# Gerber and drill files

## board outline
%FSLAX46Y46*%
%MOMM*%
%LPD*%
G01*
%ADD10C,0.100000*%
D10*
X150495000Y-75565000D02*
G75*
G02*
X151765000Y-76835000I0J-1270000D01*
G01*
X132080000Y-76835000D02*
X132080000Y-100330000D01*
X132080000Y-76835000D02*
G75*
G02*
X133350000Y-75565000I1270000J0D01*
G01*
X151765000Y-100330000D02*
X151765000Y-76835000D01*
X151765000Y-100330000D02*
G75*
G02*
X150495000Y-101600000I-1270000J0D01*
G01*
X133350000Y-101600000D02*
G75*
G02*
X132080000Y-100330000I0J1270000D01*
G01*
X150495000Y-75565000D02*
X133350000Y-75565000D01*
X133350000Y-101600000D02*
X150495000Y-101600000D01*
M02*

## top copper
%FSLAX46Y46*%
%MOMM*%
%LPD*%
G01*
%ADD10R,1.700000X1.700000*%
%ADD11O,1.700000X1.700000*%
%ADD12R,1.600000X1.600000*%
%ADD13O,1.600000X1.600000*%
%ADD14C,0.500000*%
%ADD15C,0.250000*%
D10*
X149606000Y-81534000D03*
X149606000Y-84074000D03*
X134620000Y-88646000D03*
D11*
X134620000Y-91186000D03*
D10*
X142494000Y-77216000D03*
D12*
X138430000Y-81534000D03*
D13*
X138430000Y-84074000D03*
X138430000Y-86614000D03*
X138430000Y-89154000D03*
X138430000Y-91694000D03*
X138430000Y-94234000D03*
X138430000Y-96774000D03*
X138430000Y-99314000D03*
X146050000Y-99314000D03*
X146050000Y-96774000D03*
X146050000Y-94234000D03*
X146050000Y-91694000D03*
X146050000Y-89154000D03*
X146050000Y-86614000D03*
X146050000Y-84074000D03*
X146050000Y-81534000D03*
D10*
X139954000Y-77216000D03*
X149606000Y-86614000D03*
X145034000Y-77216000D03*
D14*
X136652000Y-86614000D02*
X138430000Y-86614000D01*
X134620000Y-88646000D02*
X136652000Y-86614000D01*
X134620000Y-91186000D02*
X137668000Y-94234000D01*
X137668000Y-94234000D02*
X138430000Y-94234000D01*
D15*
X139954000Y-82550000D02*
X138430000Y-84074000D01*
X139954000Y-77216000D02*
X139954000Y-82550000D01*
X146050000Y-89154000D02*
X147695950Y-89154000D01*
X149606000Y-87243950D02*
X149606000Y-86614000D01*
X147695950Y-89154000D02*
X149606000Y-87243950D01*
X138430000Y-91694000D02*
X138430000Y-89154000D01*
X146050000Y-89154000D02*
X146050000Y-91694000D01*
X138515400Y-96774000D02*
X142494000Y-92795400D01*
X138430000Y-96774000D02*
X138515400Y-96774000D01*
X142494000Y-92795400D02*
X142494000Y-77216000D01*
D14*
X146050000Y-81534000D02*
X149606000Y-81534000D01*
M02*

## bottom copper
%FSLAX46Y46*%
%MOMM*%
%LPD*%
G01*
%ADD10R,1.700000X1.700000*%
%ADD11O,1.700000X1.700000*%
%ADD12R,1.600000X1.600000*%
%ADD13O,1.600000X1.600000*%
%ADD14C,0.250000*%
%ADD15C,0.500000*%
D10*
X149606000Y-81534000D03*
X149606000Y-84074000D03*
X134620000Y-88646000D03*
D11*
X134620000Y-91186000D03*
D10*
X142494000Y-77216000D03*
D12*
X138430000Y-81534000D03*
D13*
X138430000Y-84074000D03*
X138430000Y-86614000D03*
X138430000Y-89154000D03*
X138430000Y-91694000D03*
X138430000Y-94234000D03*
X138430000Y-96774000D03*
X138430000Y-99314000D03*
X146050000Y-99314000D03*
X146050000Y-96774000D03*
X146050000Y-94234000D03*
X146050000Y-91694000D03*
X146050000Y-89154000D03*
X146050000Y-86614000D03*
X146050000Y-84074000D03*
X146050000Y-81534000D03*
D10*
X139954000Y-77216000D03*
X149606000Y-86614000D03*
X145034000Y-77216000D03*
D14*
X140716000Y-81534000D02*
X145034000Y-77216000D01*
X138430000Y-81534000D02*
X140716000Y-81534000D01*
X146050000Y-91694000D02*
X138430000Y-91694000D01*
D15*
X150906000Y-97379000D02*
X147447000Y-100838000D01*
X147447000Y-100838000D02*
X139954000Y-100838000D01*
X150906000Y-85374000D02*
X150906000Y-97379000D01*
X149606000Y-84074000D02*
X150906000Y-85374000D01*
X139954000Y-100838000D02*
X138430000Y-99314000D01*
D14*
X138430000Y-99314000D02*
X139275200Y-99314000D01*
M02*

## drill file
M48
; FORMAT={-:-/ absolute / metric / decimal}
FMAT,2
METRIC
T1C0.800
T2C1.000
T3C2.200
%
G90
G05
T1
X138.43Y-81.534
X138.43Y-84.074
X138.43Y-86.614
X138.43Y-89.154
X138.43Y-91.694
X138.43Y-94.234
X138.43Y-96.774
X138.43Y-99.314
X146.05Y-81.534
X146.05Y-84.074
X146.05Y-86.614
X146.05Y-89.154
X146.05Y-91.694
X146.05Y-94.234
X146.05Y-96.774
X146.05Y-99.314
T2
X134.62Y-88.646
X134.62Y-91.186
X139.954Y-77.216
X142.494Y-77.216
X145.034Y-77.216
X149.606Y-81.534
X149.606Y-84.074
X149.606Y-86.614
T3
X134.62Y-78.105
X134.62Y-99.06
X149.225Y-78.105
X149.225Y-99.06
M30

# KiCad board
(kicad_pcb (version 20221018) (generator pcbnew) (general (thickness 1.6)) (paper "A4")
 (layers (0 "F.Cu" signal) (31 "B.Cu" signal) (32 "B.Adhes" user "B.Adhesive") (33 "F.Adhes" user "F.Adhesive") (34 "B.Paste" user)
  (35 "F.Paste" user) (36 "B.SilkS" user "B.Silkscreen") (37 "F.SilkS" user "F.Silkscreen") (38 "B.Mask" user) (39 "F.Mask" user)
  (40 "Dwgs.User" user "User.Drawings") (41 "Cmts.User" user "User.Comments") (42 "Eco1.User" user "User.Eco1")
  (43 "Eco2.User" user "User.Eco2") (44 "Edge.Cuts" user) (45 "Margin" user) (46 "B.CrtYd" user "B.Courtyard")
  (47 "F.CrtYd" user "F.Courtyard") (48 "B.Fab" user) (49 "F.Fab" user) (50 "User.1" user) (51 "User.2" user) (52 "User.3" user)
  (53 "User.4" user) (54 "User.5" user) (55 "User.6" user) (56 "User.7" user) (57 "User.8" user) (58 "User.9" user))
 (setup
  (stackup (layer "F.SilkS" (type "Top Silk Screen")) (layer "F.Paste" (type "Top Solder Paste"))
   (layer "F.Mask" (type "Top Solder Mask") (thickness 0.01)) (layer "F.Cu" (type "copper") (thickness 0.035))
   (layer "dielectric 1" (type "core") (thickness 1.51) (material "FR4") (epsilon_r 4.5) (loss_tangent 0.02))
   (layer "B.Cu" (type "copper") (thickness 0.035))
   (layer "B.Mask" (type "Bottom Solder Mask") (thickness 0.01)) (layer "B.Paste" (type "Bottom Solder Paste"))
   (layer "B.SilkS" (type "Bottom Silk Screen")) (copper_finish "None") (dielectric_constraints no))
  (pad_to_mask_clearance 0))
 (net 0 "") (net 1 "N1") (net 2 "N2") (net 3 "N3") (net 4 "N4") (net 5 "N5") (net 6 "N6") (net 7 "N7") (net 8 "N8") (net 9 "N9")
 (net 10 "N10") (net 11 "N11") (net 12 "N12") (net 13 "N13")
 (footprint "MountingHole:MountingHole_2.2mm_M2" (layer "F.Cu") (at 149.225 99.06)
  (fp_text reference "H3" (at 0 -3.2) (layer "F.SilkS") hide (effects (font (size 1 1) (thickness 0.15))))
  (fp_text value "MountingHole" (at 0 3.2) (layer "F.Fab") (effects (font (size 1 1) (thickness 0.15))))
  (pad "" np_thru_hole circle (at 0 0) (size 2.2 2.2) (drill 2.2) (layers "*.Cu" "*.Mask")))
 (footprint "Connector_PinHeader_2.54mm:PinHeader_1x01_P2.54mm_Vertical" (layer "F.Cu") (at 149.606 81.534)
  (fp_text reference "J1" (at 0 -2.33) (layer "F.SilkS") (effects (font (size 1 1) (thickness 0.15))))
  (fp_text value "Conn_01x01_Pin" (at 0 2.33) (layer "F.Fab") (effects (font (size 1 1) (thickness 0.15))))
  (pad "1" thru_hole rect (at 0 0) (size 1.7 1.7) (drill 1) (layers "*.Cu" "*.Mask") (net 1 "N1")))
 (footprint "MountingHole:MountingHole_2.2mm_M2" (layer "F.Cu") (at 134.62 99.06)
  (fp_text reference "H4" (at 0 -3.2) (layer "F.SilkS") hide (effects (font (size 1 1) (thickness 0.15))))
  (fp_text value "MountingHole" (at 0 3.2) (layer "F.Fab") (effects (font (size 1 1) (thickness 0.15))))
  (pad "" np_thru_hole circle (at 0 0) (size 2.2 2.2) (drill 2.2) (layers "*.Cu" "*.Mask")))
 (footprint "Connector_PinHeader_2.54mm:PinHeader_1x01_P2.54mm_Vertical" (layer "F.Cu") (at 149.606 84.074)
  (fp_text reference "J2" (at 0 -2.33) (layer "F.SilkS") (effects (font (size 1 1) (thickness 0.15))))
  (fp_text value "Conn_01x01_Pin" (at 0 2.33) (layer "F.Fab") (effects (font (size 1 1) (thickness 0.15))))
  (pad "1" thru_hole rect (at 0 0) (size 1.7 1.7) (drill 1) (layers "*.Cu" "*.Mask") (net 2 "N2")))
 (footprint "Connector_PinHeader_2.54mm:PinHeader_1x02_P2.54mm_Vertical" (layer "F.Cu") (at 134.62 88.646)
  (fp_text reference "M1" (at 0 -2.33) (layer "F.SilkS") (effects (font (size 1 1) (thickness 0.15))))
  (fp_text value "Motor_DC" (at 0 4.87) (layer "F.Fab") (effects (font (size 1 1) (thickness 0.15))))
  (pad "1" thru_hole rect (at 0 0) (size 1.7 1.7) (drill 1) (layers "*.Cu" "*.Mask") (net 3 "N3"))
  (pad "2" thru_hole oval (at 0 2.54) (size 1.7 1.7) (drill 1) (layers "*.Cu" "*.Mask") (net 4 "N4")))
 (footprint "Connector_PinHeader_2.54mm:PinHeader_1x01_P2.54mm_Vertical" (layer "F.Cu") (at 142.494 77.216)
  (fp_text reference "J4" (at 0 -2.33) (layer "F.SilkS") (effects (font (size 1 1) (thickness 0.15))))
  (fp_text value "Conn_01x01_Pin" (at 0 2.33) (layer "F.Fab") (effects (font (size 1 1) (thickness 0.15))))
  (pad "1" thru_hole rect (at 0 0) (size 1.7 1.7) (drill 1) (layers "*.Cu" "*.Mask") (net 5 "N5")))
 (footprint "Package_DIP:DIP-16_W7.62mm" (layer "F.Cu") (at 138.43 81.534)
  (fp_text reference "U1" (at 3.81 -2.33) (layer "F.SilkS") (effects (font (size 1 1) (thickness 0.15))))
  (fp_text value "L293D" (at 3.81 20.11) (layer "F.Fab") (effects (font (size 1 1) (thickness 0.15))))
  (pad "1" thru_hole rect (at 0 0) (size 1.6 1.6) (drill 0.8) (layers "*.Cu" "*.Mask") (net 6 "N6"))
  (pad "2" thru_hole oval (at 0 2.54) (size 1.6 1.6) (drill 0.8) (layers "*.Cu" "*.Mask") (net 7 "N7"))
  (pad "3" thru_hole oval (at 0 5.08) (size 1.6 1.6) (drill 0.8) (layers "*.Cu" "*.Mask") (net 3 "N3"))
  (pad "4" thru_hole oval (at 0 7.62) (size 1.6 1.6) (drill 0.8) (layers "*.Cu" "*.Mask") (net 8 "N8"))
  (pad "5" thru_hole oval (at 0 10.16) (size 1.6 1.6) (drill 0.8) (layers "*.Cu" "*.Mask") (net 8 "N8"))
  (pad "6" thru_hole oval (at 0 12.7) (size 1.6 1.6) (drill 0.8) (layers "*.Cu" "*.Mask") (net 4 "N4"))
  (pad "7" thru_hole oval (at 0 15.24) (size 1.6 1.6) (drill 0.8) (layers "*.Cu" "*.Mask") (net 5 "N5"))
  (pad "8" thru_hole oval (at 0 17.78) (size 1.6 1.6) (drill 0.8) (layers "*.Cu" "*.Mask") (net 2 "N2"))
  (pad "9" thru_hole oval (at 7.62 17.78) (size 1.6 1.6) (drill 0.8) (layers "*.Cu" "*.Mask") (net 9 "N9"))
  (pad "10" thru_hole oval (at 7.62 15.24) (size 1.6 1.6) (drill 0.8) (layers "*.Cu" "*.Mask") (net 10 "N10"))
  (pad "11" thru_hole oval (at 7.62 12.7) (size 1.6 1.6) (drill 0.8) (layers "*.Cu" "*.Mask") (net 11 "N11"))
  (pad "12" thru_hole oval (at 7.62 10.16) (size 1.6 1.6) (drill 0.8) (layers "*.Cu" "*.Mask") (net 8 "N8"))
  (pad "13" thru_hole oval (at 7.62 7.62) (size 1.6 1.6) (drill 0.8) (layers "*.Cu" "*.Mask") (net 8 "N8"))
  (pad "14" thru_hole oval (at 7.62 5.08) (size 1.6 1.6) (drill 0.8) (layers "*.Cu" "*.Mask") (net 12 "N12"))
  (pad "15" thru_hole oval (at 7.62 2.54) (size 1.6 1.6) (drill 0.8) (layers "*.Cu" "*.Mask") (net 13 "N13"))
  (pad "16" thru_hole oval (at 7.62 0) (size 1.6 1.6) (drill 0.8) (layers "*.Cu" "*.Mask") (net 1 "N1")))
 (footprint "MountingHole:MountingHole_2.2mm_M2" (layer "F.Cu") (at 134.62 78.105)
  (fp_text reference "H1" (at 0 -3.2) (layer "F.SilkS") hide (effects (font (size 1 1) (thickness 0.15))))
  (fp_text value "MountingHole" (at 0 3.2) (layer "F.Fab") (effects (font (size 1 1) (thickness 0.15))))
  (pad "" np_thru_hole circle (at 0 0) (size 2.2 2.2) (drill 2.2) (layers "*.Cu" "*.Mask")))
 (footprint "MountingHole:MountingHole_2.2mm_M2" (layer "F.Cu") (at 149.225 78.105)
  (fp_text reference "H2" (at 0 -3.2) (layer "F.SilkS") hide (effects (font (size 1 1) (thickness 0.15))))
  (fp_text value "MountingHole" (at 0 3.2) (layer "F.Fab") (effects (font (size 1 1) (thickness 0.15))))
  (pad "" np_thru_hole circle (at 0 0) (size 2.2 2.2) (drill 2.2) (layers "*.Cu" "*.Mask")))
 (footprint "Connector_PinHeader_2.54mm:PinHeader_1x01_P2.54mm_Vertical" (layer "F.Cu") (at 139.954 77.216)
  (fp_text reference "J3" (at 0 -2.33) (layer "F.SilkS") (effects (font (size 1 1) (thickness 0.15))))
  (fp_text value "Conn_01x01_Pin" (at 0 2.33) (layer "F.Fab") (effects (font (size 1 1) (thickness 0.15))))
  (pad "1" thru_hole rect (at 0 0) (size 1.7 1.7) (drill 1) (layers "*.Cu" "*.Mask") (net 7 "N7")))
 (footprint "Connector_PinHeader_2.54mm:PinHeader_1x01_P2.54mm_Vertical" (layer "F.Cu") (at 149.606 86.614)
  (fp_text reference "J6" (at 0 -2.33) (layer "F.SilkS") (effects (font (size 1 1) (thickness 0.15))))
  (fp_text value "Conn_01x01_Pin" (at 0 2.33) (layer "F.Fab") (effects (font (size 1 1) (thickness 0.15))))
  (pad "1" thru_hole rect (at 0 0) (size 1.7 1.7) (drill 1) (layers "*.Cu" "*.Mask") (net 8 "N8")))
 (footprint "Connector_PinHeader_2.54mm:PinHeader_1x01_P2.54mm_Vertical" (layer "F.Cu") (at 145.034 77.216)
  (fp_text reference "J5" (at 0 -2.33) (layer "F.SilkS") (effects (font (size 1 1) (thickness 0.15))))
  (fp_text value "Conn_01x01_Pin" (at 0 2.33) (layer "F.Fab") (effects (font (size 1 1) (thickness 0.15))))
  (pad "1" thru_hole rect (at 0 0) (size 1.7 1.7) (drill 1) (layers "*.Cu" "*.Mask") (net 6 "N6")))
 (gr_arc (start 150.495 75.565) (mid 151.393026 75.936974) (end 151.765 76.835) (stroke (width 0.1) (type default)) (layer "Edge.Cuts"))
 (gr_line (start 132.08 76.835) (end 132.08 100.33) (stroke (width 0.1) (type default)) (layer "Edge.Cuts"))
 (gr_arc (start 132.08 76.835) (mid 132.451974 75.936974) (end 133.35 75.565) (stroke (width 0.1) (type default)) (layer "Edge.Cuts"))
 (gr_line (start 151.765 100.33) (end 151.765 76.835) (stroke (width 0.1) (type default)) (layer "Edge.Cuts"))
 (gr_arc (start 151.765 100.33) (mid 151.393026 101.228026) (end 150.495 101.6) (stroke (width 0.1) (type default)) (layer "Edge.Cuts"))
 (gr_arc (start 133.35 101.6) (mid 132.451974 101.228026) (end 132.08 100.33) (stroke (width 0.1) (type default)) (layer "Edge.Cuts"))
 (gr_line (start 150.495 75.565) (end 133.35 75.565) (stroke (width 0.1) (type default)) (layer "Edge.Cuts"))
 (gr_line (start 133.35 101.6) (end 150.495 101.6) (stroke (width 0.1) (type default)) (layer "Edge.Cuts"))
 (segment (start 136.652 86.614) (end 138.43 86.614) (width 0.5) (layer "F.Cu") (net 3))
 (segment (start 134.62 88.646) (end 136.652 86.614) (width 0.5) (layer "F.Cu") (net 3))
 (segment (start 134.62 91.186) (end 137.668 94.234) (width 0.5) (layer "F.Cu") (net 4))
 (segment (start 137.668 94.234) (end 138.43 94.234) (width 0.5) (layer "F.Cu") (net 4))
 (segment (start 140.716 81.534) (end 145.034 77.216) (width 0.25) (layer "B.Cu") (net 6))
 (segment (start 138.43 81.534) (end 140.716 81.534) (width 0.25) (layer "B.Cu") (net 6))
 (segment (start 139.954 82.55) (end 138.43 84.074) (width 0.25) (layer "F.Cu") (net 7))
 (segment (start 139.954 77.216) (end 139.954 82.55) (width 0.25) (layer "F.Cu") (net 7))
 (segment (start 146.05 89.154) (end 147.69595 89.154) (width 0.25) (layer "F.Cu") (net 8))
 (segment (start 149.606 87.24395) (end 149.606 86.614) (width 0.25) (layer "F.Cu") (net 8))
 (segment (start 147.69595 89.154) (end 149.606 87.24395) (width 0.25) (layer "F.Cu") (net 8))
 (segment (start 138.43 91.694) (end 138.43 89.154) (width 0.25) (layer "F.Cu") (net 8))
 (segment (start 146.05 89.154) (end 146.05 91.694) (width 0.25) (layer "F.Cu") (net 8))
 (segment (start 146.05 91.694) (end 138.43 91.694) (width 0.25) (layer "B.Cu") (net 8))
 (segment (start 138.5154 96.774) (end 142.494 92.7954) (width 0.25) (layer "F.Cu") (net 5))
 (segment (start 138.43 96.774) (end 138.5154 96.774) (width 0.25) (layer "F.Cu") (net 5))
 (segment (start 142.494 92.7954) (end 142.494 77.216) (width 0.25) (layer "F.Cu") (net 5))
 (segment (start 150.906 97.379) (end 147.447 100.838) (width 0.5) (layer "B.Cu") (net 2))
 (segment (start 147.447 100.838) (end 139.954 100.838) (width 0.5) (layer "B.Cu") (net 2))
 (segment (start 150.906 85.374) (end 150.906 97.379) (width 0.5) (layer "B.Cu") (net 2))
 (segment (start 149.606 84.074) (end 150.906 85.374) (width 0.5) (layer "B.Cu") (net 2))
 (segment (start 139.954 100.838) (end 138.43 99.314) (width 0.5) (layer "B.Cu") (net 2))
 (segment (start 138.43 99.314) (end 139.2752 99.314) (width 0.25) (layer "B.Cu") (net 2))
 (segment (start 146.05 81.534) (end 149.606 81.534) (width 0.5) (layer "F.Cu") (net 1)))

